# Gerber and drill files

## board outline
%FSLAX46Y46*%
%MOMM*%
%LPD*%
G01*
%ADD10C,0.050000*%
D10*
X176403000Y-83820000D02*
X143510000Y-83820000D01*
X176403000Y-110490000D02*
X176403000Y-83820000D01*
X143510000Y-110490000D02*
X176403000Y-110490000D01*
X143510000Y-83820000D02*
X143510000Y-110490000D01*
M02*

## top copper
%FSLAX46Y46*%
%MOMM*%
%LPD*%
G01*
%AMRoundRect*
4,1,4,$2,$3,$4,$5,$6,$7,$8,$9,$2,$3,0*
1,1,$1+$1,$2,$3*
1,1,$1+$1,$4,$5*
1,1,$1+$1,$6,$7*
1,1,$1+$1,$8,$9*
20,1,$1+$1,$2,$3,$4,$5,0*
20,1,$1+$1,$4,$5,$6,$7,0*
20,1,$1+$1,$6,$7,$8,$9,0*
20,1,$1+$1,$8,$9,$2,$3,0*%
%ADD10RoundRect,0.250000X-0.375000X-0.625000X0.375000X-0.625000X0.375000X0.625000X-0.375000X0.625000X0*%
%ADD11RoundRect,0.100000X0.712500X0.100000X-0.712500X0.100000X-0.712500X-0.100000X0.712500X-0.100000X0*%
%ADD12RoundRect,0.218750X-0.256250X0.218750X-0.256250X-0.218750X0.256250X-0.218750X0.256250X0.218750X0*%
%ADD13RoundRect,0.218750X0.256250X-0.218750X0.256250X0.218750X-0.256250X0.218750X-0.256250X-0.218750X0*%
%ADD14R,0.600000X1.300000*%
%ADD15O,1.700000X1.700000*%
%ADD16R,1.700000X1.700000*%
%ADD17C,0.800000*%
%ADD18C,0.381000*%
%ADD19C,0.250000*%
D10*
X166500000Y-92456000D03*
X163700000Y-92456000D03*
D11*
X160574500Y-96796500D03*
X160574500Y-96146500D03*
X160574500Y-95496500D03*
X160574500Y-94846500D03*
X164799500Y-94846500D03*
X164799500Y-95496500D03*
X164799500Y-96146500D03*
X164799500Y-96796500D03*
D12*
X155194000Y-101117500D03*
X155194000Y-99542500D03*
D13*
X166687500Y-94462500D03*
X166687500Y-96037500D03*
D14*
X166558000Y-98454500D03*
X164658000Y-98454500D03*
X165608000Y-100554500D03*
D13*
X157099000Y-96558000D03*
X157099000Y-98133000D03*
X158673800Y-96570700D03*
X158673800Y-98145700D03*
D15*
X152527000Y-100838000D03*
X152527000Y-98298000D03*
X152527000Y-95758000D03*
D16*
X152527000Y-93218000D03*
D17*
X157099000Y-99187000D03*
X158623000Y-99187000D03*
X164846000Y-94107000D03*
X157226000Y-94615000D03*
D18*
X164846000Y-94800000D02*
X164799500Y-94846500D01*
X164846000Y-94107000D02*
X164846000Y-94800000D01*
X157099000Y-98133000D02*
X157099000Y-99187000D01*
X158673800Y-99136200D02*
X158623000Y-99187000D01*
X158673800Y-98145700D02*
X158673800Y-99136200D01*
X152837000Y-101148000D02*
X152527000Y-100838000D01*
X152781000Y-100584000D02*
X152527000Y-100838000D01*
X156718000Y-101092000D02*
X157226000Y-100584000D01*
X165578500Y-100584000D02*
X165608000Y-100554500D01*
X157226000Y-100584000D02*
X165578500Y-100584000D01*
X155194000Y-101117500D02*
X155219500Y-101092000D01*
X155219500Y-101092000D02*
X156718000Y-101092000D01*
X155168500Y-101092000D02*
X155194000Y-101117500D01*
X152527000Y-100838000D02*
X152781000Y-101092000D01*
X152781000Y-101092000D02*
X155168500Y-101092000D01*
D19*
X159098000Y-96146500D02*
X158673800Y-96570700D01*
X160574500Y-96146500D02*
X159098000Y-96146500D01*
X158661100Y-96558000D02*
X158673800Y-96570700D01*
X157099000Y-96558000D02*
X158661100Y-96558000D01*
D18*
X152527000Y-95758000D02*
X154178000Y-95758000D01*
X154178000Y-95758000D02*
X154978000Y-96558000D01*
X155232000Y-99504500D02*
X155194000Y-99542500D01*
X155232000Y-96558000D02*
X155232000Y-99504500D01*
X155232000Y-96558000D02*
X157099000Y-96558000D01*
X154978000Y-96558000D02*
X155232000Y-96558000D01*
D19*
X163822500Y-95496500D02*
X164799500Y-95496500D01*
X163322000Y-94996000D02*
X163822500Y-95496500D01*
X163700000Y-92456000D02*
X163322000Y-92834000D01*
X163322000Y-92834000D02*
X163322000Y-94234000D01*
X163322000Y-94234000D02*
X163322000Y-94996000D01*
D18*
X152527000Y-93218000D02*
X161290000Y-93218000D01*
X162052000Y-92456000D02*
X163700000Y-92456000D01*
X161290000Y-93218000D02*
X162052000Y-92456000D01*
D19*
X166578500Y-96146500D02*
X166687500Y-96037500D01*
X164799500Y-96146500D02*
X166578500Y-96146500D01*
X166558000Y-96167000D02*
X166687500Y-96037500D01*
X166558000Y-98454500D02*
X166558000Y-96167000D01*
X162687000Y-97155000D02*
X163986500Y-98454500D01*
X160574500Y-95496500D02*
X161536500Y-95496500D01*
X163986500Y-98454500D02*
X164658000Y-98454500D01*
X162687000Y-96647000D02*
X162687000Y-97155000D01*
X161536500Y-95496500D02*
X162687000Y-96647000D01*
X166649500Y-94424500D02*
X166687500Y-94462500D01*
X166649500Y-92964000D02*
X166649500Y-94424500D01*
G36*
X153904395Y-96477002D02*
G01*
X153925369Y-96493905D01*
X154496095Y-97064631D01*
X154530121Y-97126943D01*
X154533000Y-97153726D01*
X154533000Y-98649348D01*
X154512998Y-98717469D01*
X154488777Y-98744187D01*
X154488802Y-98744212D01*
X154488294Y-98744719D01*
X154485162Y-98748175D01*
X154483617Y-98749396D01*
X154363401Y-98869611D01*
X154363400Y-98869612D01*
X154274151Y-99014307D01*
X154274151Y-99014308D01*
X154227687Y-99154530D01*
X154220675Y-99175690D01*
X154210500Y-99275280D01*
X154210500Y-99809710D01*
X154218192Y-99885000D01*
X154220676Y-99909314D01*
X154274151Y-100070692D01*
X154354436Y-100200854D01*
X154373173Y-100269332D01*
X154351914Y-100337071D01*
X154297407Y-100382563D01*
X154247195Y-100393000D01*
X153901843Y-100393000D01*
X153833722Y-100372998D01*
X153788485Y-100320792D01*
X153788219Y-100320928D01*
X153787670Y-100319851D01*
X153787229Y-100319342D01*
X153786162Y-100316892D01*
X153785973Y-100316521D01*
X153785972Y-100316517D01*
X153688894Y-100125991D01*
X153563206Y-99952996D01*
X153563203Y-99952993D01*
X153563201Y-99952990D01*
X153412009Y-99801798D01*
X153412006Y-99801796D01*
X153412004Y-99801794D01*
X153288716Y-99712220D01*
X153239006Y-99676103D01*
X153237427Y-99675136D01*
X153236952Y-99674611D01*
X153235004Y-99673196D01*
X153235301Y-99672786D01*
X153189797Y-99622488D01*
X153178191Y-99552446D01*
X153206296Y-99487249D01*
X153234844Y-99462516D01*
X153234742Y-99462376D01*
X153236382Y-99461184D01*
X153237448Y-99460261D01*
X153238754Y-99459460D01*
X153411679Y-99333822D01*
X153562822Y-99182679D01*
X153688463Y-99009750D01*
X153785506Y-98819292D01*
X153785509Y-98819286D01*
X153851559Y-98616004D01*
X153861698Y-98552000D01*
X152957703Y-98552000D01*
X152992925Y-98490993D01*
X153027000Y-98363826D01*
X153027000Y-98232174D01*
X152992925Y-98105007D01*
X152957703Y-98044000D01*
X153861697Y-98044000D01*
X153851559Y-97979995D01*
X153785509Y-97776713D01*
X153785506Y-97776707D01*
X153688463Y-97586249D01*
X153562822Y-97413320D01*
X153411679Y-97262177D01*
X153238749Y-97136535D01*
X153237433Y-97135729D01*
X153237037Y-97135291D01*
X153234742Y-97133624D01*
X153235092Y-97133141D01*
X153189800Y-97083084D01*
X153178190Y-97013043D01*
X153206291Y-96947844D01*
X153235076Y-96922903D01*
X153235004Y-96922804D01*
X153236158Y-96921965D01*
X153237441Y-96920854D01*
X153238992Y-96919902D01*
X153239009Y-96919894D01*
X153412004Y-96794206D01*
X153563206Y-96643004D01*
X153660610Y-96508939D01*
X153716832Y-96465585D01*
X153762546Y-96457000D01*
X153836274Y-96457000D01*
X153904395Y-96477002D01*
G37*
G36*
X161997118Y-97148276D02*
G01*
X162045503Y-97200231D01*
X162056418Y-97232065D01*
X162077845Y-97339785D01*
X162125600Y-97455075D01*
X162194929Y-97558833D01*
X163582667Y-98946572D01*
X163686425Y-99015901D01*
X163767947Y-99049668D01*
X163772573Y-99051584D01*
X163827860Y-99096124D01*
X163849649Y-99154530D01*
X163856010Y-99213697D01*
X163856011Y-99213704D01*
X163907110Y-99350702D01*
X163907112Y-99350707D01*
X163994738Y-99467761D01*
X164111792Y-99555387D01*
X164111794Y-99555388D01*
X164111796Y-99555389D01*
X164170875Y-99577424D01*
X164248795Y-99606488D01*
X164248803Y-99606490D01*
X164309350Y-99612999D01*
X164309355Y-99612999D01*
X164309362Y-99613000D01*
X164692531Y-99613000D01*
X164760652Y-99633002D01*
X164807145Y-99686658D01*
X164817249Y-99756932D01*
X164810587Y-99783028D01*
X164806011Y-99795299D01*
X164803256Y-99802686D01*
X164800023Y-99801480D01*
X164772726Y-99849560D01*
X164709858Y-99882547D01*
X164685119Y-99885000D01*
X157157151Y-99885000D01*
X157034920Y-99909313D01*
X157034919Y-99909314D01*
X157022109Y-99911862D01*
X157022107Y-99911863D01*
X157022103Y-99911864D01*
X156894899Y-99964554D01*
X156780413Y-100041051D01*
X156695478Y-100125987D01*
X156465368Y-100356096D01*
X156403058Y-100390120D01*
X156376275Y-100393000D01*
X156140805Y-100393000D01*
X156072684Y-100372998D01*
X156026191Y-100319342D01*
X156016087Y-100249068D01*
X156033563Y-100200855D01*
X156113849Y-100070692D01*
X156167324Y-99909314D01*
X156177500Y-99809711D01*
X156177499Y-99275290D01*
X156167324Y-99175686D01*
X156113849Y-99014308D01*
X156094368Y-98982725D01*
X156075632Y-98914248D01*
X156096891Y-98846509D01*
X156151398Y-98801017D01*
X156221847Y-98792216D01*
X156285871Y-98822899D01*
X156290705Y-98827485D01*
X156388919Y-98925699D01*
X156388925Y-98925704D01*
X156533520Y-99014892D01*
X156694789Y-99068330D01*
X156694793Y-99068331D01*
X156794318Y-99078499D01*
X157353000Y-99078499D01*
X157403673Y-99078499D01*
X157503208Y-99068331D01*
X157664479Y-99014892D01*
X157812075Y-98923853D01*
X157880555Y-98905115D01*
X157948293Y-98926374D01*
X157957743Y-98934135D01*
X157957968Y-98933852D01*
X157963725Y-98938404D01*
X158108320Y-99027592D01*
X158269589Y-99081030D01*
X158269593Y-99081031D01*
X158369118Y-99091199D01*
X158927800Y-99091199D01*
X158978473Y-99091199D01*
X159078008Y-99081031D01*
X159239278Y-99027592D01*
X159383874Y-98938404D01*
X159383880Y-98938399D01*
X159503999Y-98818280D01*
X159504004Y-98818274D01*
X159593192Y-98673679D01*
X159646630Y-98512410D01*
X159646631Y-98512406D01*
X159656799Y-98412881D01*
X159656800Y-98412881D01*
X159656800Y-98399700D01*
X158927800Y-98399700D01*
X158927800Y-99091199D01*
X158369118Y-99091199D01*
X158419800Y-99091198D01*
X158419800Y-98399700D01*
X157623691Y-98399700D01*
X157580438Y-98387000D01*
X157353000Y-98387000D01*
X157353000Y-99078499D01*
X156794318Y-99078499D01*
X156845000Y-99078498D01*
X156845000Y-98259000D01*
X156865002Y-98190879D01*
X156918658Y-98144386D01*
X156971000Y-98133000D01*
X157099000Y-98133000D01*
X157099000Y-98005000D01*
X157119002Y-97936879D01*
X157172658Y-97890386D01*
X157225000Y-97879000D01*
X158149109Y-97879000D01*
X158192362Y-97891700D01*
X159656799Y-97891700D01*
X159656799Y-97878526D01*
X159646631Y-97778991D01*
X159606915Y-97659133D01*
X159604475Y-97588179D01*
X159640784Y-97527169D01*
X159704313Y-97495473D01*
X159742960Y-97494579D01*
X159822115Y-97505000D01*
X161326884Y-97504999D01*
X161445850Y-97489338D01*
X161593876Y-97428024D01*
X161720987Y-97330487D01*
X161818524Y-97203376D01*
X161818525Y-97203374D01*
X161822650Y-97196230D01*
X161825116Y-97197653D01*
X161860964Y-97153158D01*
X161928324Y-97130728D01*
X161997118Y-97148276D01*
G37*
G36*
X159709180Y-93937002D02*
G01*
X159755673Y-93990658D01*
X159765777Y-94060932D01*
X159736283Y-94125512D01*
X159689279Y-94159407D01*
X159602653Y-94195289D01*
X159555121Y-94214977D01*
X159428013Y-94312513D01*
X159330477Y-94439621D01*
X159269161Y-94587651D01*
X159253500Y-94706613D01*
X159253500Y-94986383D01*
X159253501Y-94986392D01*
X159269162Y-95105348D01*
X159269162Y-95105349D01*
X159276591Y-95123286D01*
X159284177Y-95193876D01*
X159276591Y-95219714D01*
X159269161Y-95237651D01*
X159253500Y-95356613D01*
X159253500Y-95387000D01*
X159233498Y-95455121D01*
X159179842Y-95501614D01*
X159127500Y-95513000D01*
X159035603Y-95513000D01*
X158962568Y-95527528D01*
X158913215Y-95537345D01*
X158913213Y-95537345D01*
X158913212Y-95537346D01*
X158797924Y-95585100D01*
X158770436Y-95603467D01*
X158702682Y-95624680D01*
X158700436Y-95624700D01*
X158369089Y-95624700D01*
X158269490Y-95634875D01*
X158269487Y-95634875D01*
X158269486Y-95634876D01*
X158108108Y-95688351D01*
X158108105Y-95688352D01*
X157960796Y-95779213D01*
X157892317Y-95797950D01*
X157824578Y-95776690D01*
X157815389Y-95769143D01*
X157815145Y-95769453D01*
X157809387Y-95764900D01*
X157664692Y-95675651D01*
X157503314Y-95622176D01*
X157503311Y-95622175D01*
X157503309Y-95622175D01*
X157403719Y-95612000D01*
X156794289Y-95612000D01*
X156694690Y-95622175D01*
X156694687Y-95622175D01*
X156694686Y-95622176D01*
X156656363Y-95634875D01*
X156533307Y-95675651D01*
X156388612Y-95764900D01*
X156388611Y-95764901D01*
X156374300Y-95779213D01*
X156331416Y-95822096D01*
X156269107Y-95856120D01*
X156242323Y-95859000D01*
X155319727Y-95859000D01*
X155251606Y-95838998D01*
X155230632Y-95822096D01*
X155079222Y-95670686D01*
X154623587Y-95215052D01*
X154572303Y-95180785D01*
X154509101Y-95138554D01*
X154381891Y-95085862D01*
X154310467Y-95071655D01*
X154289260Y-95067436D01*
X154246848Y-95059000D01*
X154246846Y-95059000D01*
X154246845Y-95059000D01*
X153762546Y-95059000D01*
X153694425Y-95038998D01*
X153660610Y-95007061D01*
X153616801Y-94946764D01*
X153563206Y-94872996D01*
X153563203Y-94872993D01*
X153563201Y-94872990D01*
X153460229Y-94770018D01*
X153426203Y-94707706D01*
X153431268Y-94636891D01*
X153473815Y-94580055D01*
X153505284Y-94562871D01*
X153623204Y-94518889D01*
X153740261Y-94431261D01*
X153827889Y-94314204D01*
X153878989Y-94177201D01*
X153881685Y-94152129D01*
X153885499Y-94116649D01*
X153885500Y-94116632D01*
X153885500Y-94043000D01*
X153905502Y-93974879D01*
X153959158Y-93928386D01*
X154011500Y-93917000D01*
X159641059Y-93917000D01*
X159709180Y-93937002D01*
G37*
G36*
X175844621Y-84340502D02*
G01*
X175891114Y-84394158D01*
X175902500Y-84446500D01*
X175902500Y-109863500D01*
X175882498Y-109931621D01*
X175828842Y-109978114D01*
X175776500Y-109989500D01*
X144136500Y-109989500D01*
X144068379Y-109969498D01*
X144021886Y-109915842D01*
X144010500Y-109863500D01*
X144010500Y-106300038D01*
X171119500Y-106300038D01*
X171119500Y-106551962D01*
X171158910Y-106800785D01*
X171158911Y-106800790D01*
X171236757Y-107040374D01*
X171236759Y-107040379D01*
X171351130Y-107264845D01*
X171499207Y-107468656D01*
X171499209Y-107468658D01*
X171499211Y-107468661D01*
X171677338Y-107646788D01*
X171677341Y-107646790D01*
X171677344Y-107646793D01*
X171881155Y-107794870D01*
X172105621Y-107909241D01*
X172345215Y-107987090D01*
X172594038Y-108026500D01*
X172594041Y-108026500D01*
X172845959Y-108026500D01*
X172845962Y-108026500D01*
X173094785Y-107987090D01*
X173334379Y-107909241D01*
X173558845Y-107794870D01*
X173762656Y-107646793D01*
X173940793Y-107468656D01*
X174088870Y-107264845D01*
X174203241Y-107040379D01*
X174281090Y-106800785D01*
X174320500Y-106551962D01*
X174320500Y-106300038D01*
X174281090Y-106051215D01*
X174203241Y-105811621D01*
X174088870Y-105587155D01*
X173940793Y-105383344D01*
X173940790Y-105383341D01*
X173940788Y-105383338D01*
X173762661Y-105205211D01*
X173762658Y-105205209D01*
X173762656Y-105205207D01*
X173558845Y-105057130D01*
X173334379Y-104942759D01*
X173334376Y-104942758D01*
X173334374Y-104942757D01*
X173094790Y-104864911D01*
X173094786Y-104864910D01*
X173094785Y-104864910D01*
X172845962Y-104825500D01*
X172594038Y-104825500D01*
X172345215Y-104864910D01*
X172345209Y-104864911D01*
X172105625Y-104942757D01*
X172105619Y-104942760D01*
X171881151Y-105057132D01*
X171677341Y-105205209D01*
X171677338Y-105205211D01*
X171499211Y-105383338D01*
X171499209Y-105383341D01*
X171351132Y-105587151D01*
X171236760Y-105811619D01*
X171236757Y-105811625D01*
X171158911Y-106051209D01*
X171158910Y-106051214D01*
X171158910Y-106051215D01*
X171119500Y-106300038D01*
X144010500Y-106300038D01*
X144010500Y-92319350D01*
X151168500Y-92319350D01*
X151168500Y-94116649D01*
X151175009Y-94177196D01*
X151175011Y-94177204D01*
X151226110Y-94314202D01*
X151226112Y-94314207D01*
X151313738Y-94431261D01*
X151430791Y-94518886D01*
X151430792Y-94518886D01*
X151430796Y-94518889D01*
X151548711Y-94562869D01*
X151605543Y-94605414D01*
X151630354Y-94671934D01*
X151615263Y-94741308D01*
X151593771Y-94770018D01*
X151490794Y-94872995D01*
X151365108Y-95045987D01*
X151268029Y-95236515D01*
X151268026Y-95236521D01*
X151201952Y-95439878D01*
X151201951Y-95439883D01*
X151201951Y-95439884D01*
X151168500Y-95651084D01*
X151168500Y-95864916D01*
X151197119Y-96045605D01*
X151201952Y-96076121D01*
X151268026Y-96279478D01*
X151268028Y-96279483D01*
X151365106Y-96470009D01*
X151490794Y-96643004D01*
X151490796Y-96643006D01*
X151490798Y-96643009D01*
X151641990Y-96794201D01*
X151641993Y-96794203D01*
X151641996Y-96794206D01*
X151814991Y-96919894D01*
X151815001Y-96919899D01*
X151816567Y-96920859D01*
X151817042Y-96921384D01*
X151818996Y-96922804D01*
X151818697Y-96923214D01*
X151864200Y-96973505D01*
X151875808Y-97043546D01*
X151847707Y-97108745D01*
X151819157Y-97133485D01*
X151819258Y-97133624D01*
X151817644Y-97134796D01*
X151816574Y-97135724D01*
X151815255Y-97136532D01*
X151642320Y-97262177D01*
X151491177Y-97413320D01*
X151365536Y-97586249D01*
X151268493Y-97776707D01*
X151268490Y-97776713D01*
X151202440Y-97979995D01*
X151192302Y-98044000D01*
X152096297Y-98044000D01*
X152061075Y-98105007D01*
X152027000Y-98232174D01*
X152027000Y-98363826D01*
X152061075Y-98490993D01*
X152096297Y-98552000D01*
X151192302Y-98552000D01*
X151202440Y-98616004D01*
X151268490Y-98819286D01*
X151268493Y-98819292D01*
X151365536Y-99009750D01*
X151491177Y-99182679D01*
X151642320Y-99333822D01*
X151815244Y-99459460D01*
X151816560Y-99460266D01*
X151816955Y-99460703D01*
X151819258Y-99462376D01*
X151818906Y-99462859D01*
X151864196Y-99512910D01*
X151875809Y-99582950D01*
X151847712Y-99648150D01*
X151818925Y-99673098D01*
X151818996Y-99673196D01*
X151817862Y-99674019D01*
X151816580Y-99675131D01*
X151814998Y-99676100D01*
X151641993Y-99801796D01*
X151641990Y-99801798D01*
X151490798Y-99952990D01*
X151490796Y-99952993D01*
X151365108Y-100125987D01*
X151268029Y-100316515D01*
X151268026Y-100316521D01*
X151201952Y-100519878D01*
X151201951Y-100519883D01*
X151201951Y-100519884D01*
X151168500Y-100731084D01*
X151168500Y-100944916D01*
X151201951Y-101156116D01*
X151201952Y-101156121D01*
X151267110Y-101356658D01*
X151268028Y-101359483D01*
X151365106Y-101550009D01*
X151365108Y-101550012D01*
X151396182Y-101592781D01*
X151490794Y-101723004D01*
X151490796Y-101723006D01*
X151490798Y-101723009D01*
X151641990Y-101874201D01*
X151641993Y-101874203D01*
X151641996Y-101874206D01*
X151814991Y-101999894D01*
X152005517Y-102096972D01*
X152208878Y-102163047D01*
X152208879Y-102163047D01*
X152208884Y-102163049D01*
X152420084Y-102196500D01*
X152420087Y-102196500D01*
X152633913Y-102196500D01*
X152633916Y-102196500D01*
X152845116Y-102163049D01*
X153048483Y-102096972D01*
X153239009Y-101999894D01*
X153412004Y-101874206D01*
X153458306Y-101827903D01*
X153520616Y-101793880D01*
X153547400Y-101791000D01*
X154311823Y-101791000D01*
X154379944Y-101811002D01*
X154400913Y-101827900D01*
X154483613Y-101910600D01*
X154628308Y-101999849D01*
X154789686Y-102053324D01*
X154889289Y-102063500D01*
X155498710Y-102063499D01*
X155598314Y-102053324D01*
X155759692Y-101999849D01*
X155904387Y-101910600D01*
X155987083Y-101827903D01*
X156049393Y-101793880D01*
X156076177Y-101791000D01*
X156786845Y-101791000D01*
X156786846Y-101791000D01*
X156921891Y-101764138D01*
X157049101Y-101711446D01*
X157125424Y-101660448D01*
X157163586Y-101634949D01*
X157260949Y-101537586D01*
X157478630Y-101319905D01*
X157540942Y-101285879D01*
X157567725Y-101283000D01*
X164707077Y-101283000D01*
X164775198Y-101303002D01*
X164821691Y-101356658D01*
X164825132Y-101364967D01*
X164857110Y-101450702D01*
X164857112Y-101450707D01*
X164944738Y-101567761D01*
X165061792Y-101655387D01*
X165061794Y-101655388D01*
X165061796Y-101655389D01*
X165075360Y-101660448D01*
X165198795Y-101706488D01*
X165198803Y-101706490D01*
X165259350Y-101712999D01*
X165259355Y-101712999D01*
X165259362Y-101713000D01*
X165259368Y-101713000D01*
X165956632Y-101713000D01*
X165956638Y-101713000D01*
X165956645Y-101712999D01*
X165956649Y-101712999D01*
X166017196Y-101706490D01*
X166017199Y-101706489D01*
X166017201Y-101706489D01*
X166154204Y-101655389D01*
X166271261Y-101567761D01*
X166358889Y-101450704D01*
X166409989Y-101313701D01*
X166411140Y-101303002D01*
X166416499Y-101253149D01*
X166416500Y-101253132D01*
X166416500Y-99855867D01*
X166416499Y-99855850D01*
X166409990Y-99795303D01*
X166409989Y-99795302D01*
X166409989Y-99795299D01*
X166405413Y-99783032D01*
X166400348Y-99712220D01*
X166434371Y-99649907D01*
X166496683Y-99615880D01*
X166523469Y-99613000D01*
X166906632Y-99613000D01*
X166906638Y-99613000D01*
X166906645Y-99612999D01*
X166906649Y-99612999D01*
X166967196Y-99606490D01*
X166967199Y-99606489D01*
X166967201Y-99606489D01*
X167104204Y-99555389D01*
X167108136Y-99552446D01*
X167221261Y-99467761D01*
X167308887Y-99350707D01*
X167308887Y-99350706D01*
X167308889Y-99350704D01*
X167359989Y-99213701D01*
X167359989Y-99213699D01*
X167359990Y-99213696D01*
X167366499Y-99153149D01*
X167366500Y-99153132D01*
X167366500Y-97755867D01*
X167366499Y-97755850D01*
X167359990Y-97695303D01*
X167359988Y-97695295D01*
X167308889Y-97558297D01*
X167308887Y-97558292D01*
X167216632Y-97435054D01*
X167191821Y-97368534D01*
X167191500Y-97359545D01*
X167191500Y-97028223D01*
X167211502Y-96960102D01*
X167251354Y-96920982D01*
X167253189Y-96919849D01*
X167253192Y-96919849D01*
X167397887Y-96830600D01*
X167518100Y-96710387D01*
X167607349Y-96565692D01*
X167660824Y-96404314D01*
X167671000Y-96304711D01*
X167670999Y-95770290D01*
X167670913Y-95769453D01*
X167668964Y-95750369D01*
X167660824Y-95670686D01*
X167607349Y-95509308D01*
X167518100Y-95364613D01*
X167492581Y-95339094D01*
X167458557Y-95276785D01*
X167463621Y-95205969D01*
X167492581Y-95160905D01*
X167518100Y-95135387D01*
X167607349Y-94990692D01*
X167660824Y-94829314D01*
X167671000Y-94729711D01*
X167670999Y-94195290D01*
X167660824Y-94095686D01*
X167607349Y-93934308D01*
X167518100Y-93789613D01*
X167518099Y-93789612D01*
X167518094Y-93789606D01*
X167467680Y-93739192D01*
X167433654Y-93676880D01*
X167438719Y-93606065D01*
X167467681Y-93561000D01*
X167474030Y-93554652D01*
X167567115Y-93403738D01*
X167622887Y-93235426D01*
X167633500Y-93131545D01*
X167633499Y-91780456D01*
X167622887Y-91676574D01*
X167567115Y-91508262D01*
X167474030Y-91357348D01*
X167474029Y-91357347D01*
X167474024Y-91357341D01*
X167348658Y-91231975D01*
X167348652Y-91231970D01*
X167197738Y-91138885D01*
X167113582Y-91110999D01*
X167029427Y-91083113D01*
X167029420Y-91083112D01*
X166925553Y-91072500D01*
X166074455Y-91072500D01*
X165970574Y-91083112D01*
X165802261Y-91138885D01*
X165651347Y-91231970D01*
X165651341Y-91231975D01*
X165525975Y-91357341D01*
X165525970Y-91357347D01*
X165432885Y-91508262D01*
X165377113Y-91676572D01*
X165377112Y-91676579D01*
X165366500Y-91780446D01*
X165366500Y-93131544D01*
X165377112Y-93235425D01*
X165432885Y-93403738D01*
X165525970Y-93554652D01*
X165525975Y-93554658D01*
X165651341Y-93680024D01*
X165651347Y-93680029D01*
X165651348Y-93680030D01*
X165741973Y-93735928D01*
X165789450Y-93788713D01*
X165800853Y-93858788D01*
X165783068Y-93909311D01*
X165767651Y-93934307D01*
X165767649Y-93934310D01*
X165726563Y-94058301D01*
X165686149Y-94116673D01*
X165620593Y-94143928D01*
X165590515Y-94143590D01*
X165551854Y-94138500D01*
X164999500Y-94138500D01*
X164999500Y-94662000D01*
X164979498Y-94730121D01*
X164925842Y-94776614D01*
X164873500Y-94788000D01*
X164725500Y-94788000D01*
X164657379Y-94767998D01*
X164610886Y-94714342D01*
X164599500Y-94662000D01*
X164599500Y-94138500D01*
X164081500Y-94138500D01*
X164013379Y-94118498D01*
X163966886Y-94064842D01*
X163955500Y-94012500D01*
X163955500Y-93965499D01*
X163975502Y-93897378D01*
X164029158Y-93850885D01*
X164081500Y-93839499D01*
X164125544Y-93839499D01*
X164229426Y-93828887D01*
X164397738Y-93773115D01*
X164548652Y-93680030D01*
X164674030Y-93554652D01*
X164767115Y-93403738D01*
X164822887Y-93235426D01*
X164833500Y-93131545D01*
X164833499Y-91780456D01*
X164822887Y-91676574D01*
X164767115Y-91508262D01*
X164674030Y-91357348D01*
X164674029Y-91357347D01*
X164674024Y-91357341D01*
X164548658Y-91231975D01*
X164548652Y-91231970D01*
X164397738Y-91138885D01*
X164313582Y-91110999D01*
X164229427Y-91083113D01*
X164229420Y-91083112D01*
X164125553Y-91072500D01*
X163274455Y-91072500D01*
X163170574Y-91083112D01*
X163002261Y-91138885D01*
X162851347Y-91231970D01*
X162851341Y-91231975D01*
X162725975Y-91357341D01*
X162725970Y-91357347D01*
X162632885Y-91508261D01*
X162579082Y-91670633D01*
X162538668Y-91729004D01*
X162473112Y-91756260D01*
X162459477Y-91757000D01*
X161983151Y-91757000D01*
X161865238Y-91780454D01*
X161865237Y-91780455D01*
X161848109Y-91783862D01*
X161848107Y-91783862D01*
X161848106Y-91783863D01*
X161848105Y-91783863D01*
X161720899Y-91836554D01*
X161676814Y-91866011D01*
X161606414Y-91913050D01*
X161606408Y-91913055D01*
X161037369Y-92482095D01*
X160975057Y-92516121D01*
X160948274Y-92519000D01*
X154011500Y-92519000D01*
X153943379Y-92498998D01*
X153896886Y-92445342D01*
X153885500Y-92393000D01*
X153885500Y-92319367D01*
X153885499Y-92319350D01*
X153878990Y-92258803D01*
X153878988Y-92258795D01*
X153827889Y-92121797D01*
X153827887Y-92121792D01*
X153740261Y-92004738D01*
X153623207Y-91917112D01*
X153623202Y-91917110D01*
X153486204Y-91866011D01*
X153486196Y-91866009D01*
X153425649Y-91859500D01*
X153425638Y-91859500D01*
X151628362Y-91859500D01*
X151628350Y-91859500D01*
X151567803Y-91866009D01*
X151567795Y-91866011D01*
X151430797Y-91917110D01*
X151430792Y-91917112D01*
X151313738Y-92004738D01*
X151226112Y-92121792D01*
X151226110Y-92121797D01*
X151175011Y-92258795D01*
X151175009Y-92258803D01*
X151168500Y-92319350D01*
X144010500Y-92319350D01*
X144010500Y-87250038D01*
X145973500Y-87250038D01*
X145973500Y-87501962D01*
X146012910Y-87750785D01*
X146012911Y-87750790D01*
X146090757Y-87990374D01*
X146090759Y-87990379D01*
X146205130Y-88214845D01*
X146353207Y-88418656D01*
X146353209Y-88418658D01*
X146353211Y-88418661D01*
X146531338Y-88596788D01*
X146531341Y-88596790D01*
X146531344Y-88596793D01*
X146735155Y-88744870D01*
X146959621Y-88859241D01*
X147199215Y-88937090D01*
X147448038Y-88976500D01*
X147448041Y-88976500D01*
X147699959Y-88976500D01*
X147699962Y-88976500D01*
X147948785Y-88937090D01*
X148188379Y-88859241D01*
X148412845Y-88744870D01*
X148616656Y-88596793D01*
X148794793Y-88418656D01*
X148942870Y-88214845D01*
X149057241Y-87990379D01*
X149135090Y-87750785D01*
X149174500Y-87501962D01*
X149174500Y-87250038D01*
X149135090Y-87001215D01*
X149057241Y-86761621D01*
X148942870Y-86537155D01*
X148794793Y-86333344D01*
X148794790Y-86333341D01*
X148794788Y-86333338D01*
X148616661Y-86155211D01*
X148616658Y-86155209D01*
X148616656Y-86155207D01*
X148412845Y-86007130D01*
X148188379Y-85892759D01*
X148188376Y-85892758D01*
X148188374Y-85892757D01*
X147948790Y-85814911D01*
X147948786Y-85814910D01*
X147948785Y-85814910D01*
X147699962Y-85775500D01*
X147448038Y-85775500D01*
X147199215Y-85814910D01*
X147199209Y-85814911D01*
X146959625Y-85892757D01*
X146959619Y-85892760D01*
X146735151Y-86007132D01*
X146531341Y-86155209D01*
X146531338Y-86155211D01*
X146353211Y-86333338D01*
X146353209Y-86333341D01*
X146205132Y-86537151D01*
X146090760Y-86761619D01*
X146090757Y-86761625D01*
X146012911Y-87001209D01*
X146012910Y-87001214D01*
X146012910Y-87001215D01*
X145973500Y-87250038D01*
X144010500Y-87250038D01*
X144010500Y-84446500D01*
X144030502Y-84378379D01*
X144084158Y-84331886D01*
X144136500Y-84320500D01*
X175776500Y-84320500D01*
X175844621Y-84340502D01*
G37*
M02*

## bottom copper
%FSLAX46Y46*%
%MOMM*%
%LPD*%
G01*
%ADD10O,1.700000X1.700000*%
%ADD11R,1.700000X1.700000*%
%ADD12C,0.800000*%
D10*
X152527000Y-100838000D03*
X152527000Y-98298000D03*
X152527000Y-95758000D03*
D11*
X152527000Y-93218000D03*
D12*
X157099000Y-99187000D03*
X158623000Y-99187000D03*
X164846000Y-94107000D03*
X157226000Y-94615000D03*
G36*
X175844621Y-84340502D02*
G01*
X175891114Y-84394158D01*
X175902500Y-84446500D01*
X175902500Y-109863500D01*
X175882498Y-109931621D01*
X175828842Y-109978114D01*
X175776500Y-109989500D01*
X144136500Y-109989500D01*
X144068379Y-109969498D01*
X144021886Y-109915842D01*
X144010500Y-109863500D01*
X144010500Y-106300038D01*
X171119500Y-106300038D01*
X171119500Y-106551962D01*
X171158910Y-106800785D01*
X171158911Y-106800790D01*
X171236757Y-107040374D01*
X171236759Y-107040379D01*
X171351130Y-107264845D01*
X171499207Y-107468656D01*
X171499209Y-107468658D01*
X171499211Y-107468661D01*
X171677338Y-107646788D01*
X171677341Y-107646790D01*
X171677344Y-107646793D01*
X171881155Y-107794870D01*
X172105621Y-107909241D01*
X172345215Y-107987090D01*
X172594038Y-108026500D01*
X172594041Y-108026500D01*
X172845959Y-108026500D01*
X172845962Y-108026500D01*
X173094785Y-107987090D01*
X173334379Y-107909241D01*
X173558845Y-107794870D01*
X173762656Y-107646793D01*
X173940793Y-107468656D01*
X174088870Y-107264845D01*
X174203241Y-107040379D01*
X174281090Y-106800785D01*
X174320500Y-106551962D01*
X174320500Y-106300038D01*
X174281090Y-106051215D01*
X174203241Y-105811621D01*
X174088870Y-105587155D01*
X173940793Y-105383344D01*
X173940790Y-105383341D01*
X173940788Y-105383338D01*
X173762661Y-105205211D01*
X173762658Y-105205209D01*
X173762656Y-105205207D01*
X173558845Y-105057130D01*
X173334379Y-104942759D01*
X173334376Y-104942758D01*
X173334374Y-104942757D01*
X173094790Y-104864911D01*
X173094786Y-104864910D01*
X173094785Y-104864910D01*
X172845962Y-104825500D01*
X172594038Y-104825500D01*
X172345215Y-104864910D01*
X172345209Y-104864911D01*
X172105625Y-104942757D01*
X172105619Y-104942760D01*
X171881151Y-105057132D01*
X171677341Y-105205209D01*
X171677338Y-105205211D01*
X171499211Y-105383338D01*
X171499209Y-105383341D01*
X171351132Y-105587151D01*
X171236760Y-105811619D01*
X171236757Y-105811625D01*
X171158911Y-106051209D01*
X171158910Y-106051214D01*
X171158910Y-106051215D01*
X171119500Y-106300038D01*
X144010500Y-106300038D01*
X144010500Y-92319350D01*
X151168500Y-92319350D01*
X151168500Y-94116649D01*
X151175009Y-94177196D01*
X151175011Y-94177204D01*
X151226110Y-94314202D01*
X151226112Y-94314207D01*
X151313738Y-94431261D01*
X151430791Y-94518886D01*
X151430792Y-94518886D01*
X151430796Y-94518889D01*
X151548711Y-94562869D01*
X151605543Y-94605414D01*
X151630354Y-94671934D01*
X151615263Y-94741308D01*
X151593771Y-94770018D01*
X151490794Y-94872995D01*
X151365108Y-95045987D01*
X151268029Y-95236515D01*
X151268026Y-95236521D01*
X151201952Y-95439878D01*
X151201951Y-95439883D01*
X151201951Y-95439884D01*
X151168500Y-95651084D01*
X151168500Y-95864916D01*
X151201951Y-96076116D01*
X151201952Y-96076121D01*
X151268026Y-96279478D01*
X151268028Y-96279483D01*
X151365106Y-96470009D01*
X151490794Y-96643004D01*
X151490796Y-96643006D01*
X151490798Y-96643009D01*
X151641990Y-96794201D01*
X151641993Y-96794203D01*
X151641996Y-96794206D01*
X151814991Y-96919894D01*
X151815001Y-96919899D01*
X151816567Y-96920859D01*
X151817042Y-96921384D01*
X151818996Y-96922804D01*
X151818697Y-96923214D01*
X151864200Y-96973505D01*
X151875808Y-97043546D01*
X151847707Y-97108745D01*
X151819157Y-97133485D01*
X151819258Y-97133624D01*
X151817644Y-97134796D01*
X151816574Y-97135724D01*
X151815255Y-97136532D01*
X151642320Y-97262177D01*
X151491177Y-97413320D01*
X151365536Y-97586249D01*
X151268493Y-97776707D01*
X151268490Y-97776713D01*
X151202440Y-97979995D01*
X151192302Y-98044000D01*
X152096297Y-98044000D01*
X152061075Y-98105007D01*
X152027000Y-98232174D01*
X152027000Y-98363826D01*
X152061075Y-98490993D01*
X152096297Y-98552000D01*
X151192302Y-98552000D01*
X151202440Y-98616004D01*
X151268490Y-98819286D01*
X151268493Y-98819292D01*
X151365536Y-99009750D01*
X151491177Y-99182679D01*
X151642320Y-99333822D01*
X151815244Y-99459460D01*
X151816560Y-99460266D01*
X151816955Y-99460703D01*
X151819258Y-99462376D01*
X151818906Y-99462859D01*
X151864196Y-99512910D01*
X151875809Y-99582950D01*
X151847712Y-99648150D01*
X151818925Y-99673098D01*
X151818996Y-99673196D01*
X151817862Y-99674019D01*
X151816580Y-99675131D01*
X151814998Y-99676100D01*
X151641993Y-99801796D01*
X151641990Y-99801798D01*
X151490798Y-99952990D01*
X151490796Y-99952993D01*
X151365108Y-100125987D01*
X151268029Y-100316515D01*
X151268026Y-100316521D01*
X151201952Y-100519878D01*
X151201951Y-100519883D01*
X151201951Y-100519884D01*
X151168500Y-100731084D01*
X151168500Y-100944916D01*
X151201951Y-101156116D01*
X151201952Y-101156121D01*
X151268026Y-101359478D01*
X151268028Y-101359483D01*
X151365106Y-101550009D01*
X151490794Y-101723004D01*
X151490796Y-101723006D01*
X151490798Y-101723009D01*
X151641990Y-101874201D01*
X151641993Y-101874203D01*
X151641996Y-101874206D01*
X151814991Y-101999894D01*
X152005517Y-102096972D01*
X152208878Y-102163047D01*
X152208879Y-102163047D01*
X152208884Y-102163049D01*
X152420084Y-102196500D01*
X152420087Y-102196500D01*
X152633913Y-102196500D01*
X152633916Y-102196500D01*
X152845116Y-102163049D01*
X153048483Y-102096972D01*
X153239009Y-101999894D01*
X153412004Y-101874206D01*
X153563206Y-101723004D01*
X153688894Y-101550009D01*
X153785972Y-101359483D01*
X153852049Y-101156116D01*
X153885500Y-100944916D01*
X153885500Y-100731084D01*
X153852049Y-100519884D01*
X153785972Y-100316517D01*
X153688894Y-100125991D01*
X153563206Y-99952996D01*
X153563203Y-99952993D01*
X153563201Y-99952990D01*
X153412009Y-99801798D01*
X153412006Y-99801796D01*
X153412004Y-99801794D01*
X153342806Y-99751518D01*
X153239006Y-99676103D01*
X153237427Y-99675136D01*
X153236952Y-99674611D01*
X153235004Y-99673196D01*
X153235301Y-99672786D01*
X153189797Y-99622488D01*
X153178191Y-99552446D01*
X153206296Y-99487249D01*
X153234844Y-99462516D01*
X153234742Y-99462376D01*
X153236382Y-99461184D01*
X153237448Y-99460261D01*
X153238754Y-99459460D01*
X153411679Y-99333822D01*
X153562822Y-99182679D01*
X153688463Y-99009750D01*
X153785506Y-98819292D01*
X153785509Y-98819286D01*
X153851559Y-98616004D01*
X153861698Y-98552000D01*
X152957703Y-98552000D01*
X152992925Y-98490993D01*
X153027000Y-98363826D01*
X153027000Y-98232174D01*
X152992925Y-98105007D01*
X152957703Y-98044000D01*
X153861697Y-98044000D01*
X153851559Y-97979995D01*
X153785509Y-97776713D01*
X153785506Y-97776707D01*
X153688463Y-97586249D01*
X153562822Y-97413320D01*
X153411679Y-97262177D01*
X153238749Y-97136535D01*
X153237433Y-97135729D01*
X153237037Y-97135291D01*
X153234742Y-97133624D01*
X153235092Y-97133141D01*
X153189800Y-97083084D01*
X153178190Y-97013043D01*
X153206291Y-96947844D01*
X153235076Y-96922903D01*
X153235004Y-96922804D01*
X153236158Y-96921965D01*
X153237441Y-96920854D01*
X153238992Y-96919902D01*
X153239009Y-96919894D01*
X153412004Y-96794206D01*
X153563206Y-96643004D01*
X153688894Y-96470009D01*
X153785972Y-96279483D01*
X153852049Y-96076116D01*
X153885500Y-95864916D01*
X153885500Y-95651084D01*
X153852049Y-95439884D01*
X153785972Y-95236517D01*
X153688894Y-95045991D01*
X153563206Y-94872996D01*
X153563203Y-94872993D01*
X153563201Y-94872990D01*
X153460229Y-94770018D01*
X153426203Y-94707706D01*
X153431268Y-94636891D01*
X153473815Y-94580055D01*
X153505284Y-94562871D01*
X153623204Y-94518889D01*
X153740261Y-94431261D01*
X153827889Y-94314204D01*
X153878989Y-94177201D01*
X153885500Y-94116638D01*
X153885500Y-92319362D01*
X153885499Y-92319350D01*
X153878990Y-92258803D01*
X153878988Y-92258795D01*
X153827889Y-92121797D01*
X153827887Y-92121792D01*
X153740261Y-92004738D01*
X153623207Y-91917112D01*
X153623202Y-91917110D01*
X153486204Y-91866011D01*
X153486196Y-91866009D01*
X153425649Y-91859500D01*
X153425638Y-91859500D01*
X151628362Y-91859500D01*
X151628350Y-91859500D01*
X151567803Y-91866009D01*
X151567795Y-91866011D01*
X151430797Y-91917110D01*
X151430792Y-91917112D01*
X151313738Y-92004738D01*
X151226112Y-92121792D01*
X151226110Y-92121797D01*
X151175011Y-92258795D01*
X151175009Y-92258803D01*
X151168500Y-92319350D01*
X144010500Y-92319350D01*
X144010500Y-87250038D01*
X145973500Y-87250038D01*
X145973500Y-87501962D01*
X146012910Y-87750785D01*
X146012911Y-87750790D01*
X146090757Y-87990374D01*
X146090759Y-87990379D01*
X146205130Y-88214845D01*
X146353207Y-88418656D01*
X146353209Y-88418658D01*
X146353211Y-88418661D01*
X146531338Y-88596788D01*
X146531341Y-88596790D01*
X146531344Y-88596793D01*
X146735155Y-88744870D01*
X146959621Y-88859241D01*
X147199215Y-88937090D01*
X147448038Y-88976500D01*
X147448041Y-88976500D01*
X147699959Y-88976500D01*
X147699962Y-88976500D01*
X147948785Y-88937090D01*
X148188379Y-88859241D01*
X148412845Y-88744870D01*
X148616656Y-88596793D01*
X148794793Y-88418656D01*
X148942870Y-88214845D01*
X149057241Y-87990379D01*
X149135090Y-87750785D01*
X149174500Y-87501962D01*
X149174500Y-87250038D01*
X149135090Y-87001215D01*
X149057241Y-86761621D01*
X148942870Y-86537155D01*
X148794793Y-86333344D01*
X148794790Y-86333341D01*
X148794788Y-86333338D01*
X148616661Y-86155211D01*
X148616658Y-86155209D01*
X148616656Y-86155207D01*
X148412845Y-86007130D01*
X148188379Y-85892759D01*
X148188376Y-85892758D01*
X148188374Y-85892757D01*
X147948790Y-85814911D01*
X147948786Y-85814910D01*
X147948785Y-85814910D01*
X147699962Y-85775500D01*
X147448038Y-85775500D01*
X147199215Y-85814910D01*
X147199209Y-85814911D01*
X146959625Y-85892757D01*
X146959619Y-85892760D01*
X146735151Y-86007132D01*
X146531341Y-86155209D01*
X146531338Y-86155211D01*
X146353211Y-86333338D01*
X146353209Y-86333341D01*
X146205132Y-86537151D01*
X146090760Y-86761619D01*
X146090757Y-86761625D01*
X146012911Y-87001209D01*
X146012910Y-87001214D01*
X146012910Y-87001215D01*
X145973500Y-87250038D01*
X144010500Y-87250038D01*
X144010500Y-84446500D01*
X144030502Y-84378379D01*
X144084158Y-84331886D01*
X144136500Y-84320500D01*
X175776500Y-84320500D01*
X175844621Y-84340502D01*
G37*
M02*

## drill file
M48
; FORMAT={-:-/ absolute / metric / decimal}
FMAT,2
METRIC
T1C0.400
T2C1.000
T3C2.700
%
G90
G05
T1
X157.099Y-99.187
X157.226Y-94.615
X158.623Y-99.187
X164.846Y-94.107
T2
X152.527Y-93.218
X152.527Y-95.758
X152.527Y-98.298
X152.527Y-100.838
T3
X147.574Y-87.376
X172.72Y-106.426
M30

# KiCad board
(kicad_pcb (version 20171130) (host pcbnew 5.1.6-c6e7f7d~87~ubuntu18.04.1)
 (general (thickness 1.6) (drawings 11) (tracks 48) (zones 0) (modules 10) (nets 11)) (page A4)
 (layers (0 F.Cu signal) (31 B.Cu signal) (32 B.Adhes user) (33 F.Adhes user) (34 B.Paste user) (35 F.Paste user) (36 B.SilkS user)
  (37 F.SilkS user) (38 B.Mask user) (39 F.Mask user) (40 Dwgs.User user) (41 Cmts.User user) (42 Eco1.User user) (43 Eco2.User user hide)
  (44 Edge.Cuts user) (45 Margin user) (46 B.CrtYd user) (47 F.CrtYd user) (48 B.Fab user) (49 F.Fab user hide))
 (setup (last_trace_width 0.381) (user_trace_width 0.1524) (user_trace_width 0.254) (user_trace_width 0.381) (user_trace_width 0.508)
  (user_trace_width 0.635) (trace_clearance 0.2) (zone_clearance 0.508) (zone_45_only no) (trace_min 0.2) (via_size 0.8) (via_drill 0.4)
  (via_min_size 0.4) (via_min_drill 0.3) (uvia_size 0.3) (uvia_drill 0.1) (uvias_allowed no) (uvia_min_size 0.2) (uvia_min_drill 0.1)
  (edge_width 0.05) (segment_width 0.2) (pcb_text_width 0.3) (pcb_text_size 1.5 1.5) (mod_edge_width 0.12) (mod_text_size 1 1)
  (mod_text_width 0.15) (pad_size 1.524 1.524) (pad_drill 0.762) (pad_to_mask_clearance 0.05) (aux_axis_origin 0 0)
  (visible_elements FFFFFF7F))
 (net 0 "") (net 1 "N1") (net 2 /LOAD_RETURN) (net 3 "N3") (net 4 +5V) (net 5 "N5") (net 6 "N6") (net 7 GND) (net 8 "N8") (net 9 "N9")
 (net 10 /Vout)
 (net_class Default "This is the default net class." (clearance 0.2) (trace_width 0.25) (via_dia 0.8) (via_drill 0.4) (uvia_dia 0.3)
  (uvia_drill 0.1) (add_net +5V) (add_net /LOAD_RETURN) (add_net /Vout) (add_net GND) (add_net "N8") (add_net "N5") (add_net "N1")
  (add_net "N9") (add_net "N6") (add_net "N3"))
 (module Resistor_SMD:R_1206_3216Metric (layer F.Cu) (at 165.1 92.456)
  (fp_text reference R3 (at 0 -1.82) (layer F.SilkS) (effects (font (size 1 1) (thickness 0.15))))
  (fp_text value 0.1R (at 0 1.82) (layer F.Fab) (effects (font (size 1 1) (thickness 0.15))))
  (pad 2 smd roundrect (at 1.4 0) (size 1.25 1.75) (layers F.Cu F.Paste F.Mask) (roundrect_rratio 0.2) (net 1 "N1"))
  (pad 1 smd roundrect (at -1.4 0) (size 1.25 1.75) (layers F.Cu F.Paste F.Mask) (roundrect_rratio 0.2) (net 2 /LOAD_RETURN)))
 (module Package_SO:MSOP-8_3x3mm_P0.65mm (layer F.Cu) (at 162.687 95.8215 180)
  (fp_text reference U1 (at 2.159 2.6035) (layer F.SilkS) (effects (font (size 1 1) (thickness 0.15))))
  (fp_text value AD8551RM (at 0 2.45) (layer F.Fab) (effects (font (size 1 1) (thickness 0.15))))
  (pad 8 smd roundrect (at 2.1125 -0.975 180) (size 1.625 0.4) (layers F.Cu F.Paste F.Mask) (roundrect_rratio 0.25) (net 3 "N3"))
  (pad 7 smd roundrect (at 2.1125 -0.325 180) (size 1.625 0.4) (layers F.Cu F.Paste F.Mask) (roundrect_rratio 0.25) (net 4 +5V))
  (pad 6 smd roundrect (at 2.1125 0.325 180) (size 1.625 0.4) (layers F.Cu F.Paste F.Mask) (roundrect_rratio 0.25) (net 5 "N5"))
  (pad 5 smd roundrect (at 2.1125 0.975 180) (size 1.625 0.4) (layers F.Cu F.Paste F.Mask) (roundrect_rratio 0.25) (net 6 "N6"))
  (pad 4 smd roundrect (at -2.1125 0.975 180) (size 1.625 0.4) (layers F.Cu F.Paste F.Mask) (roundrect_rratio 0.25) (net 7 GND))
  (pad 3 smd roundrect (at -2.1125 0.325 180) (size 1.625 0.4) (layers F.Cu F.Paste F.Mask) (roundrect_rratio 0.25) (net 2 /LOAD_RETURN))
  (pad 2 smd roundrect (at -2.1125 -0.325 180) (size 1.625 0.4) (layers F.Cu F.Paste F.Mask) (roundrect_rratio 0.25) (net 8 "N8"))
  (pad 1 smd roundrect (at -2.1125 -0.975 180) (size 1.625 0.4) (layers F.Cu F.Paste F.Mask) (roundrect_rratio 0.25) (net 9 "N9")))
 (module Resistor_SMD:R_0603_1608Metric (layer F.Cu) (at 155.194 100.33 270)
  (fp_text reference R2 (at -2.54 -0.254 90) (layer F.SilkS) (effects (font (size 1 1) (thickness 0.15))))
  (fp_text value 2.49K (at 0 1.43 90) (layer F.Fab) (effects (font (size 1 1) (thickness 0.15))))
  (pad 2 smd roundrect (at 0.7875 0 270) (size 0.875 0.95) (layers F.Cu F.Paste F.Mask) (roundrect_rratio 0.25) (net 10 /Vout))
  (pad 1 smd roundrect (at -0.7875 0 270) (size 0.875 0.95) (layers F.Cu F.Paste F.Mask) (roundrect_rratio 0.25) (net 4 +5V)))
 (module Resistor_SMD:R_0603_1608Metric (layer F.Cu) (at 166.6875 95.25 90)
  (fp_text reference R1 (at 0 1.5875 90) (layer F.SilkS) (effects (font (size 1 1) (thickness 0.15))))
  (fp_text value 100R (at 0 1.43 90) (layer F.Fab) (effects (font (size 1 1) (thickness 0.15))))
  (pad 2 smd roundrect (at 0.7875 0 90) (size 0.875 0.95) (layers F.Cu F.Paste F.Mask) (roundrect_rratio 0.25) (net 1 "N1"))
  (pad 1 smd roundrect (at -0.7875 0 90) (size 0.875 0.95) (layers F.Cu F.Paste F.Mask) (roundrect_rratio 0.25) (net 8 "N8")))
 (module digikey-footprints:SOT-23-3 (layer F.Cu) (at 165.608 99.5045 270)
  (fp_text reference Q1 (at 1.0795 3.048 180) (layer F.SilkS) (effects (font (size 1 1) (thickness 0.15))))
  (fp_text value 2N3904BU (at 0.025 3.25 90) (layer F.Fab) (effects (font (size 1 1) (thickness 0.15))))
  (pad 1 smd rect (at -1.05 -0.95 270) (size 1.3 0.6) (layers F.Cu F.Paste F.Mask) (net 8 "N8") (solder_mask_margin 0.07))
  (pad 2 smd rect (at -1.05 0.95 270) (size 1.3 0.6) (layers F.Cu F.Paste F.Mask) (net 5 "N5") (solder_mask_margin 0.07))
  (pad 3 smd rect (at 1.05 0 270) (size 1.3 0.6) (layers F.Cu F.Paste F.Mask) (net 10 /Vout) (solder_mask_margin 0.07)))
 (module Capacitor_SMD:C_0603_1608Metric (layer F.Cu) (at 157.099 97.3455 90)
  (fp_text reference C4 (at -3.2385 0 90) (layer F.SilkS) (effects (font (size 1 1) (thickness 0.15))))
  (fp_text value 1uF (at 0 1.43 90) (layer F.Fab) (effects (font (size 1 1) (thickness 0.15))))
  (pad 2 smd roundrect (at 0.7875 0 90) (size 0.875 0.95) (layers F.Cu F.Paste F.Mask) (roundrect_rratio 0.25) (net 4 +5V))
  (pad 1 smd roundrect (at -0.7875 0 90) (size 0.875 0.95) (layers F.Cu F.Paste F.Mask) (roundrect_rratio 0.25) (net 7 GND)))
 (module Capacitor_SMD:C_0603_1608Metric (layer F.Cu) (at 158.6738 97.3582 90)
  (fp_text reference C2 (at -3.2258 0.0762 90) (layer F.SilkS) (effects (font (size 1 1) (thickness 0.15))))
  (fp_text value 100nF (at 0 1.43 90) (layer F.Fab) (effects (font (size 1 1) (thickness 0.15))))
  (pad 2 smd roundrect (at 0.7875 0 90) (size 0.875 0.95) (layers F.Cu F.Paste F.Mask) (roundrect_rratio 0.25) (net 4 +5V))
  (pad 1 smd roundrect (at -0.7875 0 90) (size 0.875 0.95) (layers F.Cu F.Paste F.Mask) (roundrect_rratio 0.25) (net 7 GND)))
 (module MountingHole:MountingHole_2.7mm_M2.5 (layer F.Cu) (at 172.72 106.426)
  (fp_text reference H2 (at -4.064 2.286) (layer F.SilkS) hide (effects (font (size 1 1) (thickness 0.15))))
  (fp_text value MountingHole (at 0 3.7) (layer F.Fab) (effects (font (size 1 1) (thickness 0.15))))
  (pad 1 np_thru_hole circle (at 0 0) (size 2.7 2.7) (drill 2.7) (layers *.Cu *.Mask)))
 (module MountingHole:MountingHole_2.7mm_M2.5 (layer F.Cu) (at 147.574 87.376)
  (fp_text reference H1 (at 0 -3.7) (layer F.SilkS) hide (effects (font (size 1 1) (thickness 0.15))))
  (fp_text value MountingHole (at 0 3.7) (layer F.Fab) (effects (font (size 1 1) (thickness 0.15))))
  (pad 1 np_thru_hole circle (at 0 0) (size 2.7 2.7) (drill 2.7) (layers *.Cu *.Mask)))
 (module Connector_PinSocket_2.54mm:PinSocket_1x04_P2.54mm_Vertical (layer F.Cu) (at 152.527 93.218)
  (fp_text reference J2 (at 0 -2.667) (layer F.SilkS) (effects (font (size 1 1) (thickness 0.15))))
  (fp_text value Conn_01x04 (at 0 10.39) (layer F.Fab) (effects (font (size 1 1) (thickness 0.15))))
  (pad 4 thru_hole oval (at 0 7.62) (size 1.7 1.7) (drill 1) (layers *.Cu *.Mask) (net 10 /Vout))
  (pad 3 thru_hole oval (at 0 5.08) (size 1.7 1.7) (drill 1) (layers *.Cu *.Mask) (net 7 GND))
  (pad 2 thru_hole oval (at 0 2.54) (size 1.7 1.7) (drill 1) (layers *.Cu *.Mask) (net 4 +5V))
  (pad 1 thru_hole rect (at 0 0) (size 1.7 1.7) (drill 1) (layers *.Cu *.Mask) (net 2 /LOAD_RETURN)))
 (gr_line (start 176.403 83.82) (end 143.51 83.82) (layer Edge.Cuts) (width 0.05))
 (gr_line (start 176.403 110.49) (end 176.403 83.82) (layer Edge.Cuts) (width 0.05))
 (gr_line (start 143.51 110.49) (end 176.403 110.49) (layer Edge.Cuts) (width 0.05))
 (gr_line (start 143.51 83.82) (end 143.51 110.49) (layer Edge.Cuts) (width 0.05))
 (via (at 157.099 99.187) (size 0.8) (drill 0.4) (layers F.Cu B.Cu) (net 7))
 (via (at 158.623 99.187) (size 0.8) (drill 0.4) (layers F.Cu B.Cu) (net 7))
 (via (at 164.846 94.107) (size 0.8) (drill 0.4) (layers F.Cu B.Cu) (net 7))
 (segment (start 164.846 94.8) (end 164.7995 94.8465) (width 0.381) (layer F.Cu) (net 7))
 (segment (start 164.846 94.107) (end 164.846 94.8) (width 0.381) (layer F.Cu) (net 7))
 (segment (start 157.099 98.133) (end 157.099 99.187) (width 0.381) (layer F.Cu) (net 7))
 (segment (start 158.6738 99.1362) (end 158.623 99.187) (width 0.381) (layer F.Cu) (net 7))
 (segment (start 158.6738 98.1457) (end 158.6738 99.1362) (width 0.381) (layer F.Cu) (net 7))
 (via (at 157.226 94.615) (size 0.8) (drill 0.4) (layers F.Cu B.Cu) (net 7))
 (segment (start 152.837 101.148) (end 152.527 100.838) (width 0.381) (layer F.Cu) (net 10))
 (segment (start 152.781 100.584) (end 152.527 100.838) (width 0.381) (layer F.Cu) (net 10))
 (segment (start 156.718 101.092) (end 157.226 100.584) (width 0.381) (layer F.Cu) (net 10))
 (segment (start 165.5785 100.584) (end 165.608 100.5545) (width 0.381) (layer F.Cu) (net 10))
 (segment (start 157.226 100.584) (end 165.5785 100.584) (width 0.381) (layer F.Cu) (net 10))
 (segment (start 155.194 101.1175) (end 155.2195 101.092) (width 0.381) (layer F.Cu) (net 10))
 (segment (start 155.2195 101.092) (end 156.718 101.092) (width 0.381) (layer F.Cu) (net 10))
 (segment (start 155.1685 101.092) (end 155.194 101.1175) (width 0.381) (layer F.Cu) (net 10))
 (segment (start 152.527 100.838) (end 152.781 101.092) (width 0.381) (layer F.Cu) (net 10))
 (segment (start 152.781 101.092) (end 155.1685 101.092) (width 0.381) (layer F.Cu) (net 10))
 (segment (start 159.098 96.1465) (end 158.6738 96.5707) (width 0.25) (layer F.Cu) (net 4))
 (segment (start 160.5745 96.1465) (end 159.098 96.1465) (width 0.25) (layer F.Cu) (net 4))
 (segment (start 158.6611 96.558) (end 158.6738 96.5707) (width 0.25) (layer F.Cu) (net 4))
 (segment (start 157.099 96.558) (end 158.6611 96.558) (width 0.25) (layer F.Cu) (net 4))
 (segment (start 152.527 95.758) (end 154.178 95.758) (width 0.381) (layer F.Cu) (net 4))
 (segment (start 154.178 95.758) (end 154.978 96.558) (width 0.381) (layer F.Cu) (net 4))
 (segment (start 155.232 99.5045) (end 155.194 99.5425) (width 0.381) (layer F.Cu) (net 4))
 (segment (start 155.232 96.558) (end 155.232 99.5045) (width 0.381) (layer F.Cu) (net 4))
 (segment (start 155.232 96.558) (end 157.099 96.558) (width 0.381) (layer F.Cu) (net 4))
 (segment (start 154.978 96.558) (end 155.232 96.558) (width 0.381) (layer F.Cu) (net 4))
 (segment (start 163.8225 95.4965) (end 164.7995 95.4965) (width 0.25) (layer F.Cu) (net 2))
 (segment (start 163.322 94.996) (end 163.8225 95.4965) (width 0.25) (layer F.Cu) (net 2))
 (segment (start 163.7 92.456) (end 163.322 92.834) (width 0.25) (layer F.Cu) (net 2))
 (segment (start 163.322 92.834) (end 163.322 94.234) (width 0.25) (layer F.Cu) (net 2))
 (segment (start 163.322 94.234) (end 163.322 94.996) (width 0.25) (layer F.Cu) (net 2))
 (segment (start 152.527 93.218) (end 161.29 93.218) (width 0.381) (layer F.Cu) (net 2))
 (segment (start 162.052 92.456) (end 163.7 92.456) (width 0.381) (layer F.Cu) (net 2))
 (segment (start 161.29 93.218) (end 162.052 92.456) (width 0.381) (layer F.Cu) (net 2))
 (segment (start 166.5785 96.1465) (end 166.6875 96.0375) (width 0.25) (layer F.Cu) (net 8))
 (segment (start 164.7995 96.1465) (end 166.5785 96.1465) (width 0.25) (layer F.Cu) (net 8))
 (segment (start 166.558 96.167) (end 166.6875 96.0375) (width 0.25) (layer F.Cu) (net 8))
 (segment (start 166.558 98.4545) (end 166.558 96.167) (width 0.25) (layer F.Cu) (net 8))
 (segment (start 162.687 97.155) (end 163.9865 98.4545) (width 0.25) (layer F.Cu) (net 5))
 (segment (start 160.5745 95.4965) (end 161.5365 95.4965) (width 0.25) (layer F.Cu) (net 5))
 (segment (start 163.9865 98.4545) (end 164.658 98.4545) (width 0.25) (layer F.Cu) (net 5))
 (segment (start 162.687 96.647) (end 162.687 97.155) (width 0.25) (layer F.Cu) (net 5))
 (segment (start 161.5365 95.4965) (end 162.687 96.647) (width 0.25) (layer F.Cu) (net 5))
 (segment (start 166.6495 94.4245) (end 166.6875 94.4625) (width 0.25) (layer F.Cu) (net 1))
 (segment (start 166.6495 92.964) (end 166.6495 94.4245) (width 0.25) (layer F.Cu) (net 1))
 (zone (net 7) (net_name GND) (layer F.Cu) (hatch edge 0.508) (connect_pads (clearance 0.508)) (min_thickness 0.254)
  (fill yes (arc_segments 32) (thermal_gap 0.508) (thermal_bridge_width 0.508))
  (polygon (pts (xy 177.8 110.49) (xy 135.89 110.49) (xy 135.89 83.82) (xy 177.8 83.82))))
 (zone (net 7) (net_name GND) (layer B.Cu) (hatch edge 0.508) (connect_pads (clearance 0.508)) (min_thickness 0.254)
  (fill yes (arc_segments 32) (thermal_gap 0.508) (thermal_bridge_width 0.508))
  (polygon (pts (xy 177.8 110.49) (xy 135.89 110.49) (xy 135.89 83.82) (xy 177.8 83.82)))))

